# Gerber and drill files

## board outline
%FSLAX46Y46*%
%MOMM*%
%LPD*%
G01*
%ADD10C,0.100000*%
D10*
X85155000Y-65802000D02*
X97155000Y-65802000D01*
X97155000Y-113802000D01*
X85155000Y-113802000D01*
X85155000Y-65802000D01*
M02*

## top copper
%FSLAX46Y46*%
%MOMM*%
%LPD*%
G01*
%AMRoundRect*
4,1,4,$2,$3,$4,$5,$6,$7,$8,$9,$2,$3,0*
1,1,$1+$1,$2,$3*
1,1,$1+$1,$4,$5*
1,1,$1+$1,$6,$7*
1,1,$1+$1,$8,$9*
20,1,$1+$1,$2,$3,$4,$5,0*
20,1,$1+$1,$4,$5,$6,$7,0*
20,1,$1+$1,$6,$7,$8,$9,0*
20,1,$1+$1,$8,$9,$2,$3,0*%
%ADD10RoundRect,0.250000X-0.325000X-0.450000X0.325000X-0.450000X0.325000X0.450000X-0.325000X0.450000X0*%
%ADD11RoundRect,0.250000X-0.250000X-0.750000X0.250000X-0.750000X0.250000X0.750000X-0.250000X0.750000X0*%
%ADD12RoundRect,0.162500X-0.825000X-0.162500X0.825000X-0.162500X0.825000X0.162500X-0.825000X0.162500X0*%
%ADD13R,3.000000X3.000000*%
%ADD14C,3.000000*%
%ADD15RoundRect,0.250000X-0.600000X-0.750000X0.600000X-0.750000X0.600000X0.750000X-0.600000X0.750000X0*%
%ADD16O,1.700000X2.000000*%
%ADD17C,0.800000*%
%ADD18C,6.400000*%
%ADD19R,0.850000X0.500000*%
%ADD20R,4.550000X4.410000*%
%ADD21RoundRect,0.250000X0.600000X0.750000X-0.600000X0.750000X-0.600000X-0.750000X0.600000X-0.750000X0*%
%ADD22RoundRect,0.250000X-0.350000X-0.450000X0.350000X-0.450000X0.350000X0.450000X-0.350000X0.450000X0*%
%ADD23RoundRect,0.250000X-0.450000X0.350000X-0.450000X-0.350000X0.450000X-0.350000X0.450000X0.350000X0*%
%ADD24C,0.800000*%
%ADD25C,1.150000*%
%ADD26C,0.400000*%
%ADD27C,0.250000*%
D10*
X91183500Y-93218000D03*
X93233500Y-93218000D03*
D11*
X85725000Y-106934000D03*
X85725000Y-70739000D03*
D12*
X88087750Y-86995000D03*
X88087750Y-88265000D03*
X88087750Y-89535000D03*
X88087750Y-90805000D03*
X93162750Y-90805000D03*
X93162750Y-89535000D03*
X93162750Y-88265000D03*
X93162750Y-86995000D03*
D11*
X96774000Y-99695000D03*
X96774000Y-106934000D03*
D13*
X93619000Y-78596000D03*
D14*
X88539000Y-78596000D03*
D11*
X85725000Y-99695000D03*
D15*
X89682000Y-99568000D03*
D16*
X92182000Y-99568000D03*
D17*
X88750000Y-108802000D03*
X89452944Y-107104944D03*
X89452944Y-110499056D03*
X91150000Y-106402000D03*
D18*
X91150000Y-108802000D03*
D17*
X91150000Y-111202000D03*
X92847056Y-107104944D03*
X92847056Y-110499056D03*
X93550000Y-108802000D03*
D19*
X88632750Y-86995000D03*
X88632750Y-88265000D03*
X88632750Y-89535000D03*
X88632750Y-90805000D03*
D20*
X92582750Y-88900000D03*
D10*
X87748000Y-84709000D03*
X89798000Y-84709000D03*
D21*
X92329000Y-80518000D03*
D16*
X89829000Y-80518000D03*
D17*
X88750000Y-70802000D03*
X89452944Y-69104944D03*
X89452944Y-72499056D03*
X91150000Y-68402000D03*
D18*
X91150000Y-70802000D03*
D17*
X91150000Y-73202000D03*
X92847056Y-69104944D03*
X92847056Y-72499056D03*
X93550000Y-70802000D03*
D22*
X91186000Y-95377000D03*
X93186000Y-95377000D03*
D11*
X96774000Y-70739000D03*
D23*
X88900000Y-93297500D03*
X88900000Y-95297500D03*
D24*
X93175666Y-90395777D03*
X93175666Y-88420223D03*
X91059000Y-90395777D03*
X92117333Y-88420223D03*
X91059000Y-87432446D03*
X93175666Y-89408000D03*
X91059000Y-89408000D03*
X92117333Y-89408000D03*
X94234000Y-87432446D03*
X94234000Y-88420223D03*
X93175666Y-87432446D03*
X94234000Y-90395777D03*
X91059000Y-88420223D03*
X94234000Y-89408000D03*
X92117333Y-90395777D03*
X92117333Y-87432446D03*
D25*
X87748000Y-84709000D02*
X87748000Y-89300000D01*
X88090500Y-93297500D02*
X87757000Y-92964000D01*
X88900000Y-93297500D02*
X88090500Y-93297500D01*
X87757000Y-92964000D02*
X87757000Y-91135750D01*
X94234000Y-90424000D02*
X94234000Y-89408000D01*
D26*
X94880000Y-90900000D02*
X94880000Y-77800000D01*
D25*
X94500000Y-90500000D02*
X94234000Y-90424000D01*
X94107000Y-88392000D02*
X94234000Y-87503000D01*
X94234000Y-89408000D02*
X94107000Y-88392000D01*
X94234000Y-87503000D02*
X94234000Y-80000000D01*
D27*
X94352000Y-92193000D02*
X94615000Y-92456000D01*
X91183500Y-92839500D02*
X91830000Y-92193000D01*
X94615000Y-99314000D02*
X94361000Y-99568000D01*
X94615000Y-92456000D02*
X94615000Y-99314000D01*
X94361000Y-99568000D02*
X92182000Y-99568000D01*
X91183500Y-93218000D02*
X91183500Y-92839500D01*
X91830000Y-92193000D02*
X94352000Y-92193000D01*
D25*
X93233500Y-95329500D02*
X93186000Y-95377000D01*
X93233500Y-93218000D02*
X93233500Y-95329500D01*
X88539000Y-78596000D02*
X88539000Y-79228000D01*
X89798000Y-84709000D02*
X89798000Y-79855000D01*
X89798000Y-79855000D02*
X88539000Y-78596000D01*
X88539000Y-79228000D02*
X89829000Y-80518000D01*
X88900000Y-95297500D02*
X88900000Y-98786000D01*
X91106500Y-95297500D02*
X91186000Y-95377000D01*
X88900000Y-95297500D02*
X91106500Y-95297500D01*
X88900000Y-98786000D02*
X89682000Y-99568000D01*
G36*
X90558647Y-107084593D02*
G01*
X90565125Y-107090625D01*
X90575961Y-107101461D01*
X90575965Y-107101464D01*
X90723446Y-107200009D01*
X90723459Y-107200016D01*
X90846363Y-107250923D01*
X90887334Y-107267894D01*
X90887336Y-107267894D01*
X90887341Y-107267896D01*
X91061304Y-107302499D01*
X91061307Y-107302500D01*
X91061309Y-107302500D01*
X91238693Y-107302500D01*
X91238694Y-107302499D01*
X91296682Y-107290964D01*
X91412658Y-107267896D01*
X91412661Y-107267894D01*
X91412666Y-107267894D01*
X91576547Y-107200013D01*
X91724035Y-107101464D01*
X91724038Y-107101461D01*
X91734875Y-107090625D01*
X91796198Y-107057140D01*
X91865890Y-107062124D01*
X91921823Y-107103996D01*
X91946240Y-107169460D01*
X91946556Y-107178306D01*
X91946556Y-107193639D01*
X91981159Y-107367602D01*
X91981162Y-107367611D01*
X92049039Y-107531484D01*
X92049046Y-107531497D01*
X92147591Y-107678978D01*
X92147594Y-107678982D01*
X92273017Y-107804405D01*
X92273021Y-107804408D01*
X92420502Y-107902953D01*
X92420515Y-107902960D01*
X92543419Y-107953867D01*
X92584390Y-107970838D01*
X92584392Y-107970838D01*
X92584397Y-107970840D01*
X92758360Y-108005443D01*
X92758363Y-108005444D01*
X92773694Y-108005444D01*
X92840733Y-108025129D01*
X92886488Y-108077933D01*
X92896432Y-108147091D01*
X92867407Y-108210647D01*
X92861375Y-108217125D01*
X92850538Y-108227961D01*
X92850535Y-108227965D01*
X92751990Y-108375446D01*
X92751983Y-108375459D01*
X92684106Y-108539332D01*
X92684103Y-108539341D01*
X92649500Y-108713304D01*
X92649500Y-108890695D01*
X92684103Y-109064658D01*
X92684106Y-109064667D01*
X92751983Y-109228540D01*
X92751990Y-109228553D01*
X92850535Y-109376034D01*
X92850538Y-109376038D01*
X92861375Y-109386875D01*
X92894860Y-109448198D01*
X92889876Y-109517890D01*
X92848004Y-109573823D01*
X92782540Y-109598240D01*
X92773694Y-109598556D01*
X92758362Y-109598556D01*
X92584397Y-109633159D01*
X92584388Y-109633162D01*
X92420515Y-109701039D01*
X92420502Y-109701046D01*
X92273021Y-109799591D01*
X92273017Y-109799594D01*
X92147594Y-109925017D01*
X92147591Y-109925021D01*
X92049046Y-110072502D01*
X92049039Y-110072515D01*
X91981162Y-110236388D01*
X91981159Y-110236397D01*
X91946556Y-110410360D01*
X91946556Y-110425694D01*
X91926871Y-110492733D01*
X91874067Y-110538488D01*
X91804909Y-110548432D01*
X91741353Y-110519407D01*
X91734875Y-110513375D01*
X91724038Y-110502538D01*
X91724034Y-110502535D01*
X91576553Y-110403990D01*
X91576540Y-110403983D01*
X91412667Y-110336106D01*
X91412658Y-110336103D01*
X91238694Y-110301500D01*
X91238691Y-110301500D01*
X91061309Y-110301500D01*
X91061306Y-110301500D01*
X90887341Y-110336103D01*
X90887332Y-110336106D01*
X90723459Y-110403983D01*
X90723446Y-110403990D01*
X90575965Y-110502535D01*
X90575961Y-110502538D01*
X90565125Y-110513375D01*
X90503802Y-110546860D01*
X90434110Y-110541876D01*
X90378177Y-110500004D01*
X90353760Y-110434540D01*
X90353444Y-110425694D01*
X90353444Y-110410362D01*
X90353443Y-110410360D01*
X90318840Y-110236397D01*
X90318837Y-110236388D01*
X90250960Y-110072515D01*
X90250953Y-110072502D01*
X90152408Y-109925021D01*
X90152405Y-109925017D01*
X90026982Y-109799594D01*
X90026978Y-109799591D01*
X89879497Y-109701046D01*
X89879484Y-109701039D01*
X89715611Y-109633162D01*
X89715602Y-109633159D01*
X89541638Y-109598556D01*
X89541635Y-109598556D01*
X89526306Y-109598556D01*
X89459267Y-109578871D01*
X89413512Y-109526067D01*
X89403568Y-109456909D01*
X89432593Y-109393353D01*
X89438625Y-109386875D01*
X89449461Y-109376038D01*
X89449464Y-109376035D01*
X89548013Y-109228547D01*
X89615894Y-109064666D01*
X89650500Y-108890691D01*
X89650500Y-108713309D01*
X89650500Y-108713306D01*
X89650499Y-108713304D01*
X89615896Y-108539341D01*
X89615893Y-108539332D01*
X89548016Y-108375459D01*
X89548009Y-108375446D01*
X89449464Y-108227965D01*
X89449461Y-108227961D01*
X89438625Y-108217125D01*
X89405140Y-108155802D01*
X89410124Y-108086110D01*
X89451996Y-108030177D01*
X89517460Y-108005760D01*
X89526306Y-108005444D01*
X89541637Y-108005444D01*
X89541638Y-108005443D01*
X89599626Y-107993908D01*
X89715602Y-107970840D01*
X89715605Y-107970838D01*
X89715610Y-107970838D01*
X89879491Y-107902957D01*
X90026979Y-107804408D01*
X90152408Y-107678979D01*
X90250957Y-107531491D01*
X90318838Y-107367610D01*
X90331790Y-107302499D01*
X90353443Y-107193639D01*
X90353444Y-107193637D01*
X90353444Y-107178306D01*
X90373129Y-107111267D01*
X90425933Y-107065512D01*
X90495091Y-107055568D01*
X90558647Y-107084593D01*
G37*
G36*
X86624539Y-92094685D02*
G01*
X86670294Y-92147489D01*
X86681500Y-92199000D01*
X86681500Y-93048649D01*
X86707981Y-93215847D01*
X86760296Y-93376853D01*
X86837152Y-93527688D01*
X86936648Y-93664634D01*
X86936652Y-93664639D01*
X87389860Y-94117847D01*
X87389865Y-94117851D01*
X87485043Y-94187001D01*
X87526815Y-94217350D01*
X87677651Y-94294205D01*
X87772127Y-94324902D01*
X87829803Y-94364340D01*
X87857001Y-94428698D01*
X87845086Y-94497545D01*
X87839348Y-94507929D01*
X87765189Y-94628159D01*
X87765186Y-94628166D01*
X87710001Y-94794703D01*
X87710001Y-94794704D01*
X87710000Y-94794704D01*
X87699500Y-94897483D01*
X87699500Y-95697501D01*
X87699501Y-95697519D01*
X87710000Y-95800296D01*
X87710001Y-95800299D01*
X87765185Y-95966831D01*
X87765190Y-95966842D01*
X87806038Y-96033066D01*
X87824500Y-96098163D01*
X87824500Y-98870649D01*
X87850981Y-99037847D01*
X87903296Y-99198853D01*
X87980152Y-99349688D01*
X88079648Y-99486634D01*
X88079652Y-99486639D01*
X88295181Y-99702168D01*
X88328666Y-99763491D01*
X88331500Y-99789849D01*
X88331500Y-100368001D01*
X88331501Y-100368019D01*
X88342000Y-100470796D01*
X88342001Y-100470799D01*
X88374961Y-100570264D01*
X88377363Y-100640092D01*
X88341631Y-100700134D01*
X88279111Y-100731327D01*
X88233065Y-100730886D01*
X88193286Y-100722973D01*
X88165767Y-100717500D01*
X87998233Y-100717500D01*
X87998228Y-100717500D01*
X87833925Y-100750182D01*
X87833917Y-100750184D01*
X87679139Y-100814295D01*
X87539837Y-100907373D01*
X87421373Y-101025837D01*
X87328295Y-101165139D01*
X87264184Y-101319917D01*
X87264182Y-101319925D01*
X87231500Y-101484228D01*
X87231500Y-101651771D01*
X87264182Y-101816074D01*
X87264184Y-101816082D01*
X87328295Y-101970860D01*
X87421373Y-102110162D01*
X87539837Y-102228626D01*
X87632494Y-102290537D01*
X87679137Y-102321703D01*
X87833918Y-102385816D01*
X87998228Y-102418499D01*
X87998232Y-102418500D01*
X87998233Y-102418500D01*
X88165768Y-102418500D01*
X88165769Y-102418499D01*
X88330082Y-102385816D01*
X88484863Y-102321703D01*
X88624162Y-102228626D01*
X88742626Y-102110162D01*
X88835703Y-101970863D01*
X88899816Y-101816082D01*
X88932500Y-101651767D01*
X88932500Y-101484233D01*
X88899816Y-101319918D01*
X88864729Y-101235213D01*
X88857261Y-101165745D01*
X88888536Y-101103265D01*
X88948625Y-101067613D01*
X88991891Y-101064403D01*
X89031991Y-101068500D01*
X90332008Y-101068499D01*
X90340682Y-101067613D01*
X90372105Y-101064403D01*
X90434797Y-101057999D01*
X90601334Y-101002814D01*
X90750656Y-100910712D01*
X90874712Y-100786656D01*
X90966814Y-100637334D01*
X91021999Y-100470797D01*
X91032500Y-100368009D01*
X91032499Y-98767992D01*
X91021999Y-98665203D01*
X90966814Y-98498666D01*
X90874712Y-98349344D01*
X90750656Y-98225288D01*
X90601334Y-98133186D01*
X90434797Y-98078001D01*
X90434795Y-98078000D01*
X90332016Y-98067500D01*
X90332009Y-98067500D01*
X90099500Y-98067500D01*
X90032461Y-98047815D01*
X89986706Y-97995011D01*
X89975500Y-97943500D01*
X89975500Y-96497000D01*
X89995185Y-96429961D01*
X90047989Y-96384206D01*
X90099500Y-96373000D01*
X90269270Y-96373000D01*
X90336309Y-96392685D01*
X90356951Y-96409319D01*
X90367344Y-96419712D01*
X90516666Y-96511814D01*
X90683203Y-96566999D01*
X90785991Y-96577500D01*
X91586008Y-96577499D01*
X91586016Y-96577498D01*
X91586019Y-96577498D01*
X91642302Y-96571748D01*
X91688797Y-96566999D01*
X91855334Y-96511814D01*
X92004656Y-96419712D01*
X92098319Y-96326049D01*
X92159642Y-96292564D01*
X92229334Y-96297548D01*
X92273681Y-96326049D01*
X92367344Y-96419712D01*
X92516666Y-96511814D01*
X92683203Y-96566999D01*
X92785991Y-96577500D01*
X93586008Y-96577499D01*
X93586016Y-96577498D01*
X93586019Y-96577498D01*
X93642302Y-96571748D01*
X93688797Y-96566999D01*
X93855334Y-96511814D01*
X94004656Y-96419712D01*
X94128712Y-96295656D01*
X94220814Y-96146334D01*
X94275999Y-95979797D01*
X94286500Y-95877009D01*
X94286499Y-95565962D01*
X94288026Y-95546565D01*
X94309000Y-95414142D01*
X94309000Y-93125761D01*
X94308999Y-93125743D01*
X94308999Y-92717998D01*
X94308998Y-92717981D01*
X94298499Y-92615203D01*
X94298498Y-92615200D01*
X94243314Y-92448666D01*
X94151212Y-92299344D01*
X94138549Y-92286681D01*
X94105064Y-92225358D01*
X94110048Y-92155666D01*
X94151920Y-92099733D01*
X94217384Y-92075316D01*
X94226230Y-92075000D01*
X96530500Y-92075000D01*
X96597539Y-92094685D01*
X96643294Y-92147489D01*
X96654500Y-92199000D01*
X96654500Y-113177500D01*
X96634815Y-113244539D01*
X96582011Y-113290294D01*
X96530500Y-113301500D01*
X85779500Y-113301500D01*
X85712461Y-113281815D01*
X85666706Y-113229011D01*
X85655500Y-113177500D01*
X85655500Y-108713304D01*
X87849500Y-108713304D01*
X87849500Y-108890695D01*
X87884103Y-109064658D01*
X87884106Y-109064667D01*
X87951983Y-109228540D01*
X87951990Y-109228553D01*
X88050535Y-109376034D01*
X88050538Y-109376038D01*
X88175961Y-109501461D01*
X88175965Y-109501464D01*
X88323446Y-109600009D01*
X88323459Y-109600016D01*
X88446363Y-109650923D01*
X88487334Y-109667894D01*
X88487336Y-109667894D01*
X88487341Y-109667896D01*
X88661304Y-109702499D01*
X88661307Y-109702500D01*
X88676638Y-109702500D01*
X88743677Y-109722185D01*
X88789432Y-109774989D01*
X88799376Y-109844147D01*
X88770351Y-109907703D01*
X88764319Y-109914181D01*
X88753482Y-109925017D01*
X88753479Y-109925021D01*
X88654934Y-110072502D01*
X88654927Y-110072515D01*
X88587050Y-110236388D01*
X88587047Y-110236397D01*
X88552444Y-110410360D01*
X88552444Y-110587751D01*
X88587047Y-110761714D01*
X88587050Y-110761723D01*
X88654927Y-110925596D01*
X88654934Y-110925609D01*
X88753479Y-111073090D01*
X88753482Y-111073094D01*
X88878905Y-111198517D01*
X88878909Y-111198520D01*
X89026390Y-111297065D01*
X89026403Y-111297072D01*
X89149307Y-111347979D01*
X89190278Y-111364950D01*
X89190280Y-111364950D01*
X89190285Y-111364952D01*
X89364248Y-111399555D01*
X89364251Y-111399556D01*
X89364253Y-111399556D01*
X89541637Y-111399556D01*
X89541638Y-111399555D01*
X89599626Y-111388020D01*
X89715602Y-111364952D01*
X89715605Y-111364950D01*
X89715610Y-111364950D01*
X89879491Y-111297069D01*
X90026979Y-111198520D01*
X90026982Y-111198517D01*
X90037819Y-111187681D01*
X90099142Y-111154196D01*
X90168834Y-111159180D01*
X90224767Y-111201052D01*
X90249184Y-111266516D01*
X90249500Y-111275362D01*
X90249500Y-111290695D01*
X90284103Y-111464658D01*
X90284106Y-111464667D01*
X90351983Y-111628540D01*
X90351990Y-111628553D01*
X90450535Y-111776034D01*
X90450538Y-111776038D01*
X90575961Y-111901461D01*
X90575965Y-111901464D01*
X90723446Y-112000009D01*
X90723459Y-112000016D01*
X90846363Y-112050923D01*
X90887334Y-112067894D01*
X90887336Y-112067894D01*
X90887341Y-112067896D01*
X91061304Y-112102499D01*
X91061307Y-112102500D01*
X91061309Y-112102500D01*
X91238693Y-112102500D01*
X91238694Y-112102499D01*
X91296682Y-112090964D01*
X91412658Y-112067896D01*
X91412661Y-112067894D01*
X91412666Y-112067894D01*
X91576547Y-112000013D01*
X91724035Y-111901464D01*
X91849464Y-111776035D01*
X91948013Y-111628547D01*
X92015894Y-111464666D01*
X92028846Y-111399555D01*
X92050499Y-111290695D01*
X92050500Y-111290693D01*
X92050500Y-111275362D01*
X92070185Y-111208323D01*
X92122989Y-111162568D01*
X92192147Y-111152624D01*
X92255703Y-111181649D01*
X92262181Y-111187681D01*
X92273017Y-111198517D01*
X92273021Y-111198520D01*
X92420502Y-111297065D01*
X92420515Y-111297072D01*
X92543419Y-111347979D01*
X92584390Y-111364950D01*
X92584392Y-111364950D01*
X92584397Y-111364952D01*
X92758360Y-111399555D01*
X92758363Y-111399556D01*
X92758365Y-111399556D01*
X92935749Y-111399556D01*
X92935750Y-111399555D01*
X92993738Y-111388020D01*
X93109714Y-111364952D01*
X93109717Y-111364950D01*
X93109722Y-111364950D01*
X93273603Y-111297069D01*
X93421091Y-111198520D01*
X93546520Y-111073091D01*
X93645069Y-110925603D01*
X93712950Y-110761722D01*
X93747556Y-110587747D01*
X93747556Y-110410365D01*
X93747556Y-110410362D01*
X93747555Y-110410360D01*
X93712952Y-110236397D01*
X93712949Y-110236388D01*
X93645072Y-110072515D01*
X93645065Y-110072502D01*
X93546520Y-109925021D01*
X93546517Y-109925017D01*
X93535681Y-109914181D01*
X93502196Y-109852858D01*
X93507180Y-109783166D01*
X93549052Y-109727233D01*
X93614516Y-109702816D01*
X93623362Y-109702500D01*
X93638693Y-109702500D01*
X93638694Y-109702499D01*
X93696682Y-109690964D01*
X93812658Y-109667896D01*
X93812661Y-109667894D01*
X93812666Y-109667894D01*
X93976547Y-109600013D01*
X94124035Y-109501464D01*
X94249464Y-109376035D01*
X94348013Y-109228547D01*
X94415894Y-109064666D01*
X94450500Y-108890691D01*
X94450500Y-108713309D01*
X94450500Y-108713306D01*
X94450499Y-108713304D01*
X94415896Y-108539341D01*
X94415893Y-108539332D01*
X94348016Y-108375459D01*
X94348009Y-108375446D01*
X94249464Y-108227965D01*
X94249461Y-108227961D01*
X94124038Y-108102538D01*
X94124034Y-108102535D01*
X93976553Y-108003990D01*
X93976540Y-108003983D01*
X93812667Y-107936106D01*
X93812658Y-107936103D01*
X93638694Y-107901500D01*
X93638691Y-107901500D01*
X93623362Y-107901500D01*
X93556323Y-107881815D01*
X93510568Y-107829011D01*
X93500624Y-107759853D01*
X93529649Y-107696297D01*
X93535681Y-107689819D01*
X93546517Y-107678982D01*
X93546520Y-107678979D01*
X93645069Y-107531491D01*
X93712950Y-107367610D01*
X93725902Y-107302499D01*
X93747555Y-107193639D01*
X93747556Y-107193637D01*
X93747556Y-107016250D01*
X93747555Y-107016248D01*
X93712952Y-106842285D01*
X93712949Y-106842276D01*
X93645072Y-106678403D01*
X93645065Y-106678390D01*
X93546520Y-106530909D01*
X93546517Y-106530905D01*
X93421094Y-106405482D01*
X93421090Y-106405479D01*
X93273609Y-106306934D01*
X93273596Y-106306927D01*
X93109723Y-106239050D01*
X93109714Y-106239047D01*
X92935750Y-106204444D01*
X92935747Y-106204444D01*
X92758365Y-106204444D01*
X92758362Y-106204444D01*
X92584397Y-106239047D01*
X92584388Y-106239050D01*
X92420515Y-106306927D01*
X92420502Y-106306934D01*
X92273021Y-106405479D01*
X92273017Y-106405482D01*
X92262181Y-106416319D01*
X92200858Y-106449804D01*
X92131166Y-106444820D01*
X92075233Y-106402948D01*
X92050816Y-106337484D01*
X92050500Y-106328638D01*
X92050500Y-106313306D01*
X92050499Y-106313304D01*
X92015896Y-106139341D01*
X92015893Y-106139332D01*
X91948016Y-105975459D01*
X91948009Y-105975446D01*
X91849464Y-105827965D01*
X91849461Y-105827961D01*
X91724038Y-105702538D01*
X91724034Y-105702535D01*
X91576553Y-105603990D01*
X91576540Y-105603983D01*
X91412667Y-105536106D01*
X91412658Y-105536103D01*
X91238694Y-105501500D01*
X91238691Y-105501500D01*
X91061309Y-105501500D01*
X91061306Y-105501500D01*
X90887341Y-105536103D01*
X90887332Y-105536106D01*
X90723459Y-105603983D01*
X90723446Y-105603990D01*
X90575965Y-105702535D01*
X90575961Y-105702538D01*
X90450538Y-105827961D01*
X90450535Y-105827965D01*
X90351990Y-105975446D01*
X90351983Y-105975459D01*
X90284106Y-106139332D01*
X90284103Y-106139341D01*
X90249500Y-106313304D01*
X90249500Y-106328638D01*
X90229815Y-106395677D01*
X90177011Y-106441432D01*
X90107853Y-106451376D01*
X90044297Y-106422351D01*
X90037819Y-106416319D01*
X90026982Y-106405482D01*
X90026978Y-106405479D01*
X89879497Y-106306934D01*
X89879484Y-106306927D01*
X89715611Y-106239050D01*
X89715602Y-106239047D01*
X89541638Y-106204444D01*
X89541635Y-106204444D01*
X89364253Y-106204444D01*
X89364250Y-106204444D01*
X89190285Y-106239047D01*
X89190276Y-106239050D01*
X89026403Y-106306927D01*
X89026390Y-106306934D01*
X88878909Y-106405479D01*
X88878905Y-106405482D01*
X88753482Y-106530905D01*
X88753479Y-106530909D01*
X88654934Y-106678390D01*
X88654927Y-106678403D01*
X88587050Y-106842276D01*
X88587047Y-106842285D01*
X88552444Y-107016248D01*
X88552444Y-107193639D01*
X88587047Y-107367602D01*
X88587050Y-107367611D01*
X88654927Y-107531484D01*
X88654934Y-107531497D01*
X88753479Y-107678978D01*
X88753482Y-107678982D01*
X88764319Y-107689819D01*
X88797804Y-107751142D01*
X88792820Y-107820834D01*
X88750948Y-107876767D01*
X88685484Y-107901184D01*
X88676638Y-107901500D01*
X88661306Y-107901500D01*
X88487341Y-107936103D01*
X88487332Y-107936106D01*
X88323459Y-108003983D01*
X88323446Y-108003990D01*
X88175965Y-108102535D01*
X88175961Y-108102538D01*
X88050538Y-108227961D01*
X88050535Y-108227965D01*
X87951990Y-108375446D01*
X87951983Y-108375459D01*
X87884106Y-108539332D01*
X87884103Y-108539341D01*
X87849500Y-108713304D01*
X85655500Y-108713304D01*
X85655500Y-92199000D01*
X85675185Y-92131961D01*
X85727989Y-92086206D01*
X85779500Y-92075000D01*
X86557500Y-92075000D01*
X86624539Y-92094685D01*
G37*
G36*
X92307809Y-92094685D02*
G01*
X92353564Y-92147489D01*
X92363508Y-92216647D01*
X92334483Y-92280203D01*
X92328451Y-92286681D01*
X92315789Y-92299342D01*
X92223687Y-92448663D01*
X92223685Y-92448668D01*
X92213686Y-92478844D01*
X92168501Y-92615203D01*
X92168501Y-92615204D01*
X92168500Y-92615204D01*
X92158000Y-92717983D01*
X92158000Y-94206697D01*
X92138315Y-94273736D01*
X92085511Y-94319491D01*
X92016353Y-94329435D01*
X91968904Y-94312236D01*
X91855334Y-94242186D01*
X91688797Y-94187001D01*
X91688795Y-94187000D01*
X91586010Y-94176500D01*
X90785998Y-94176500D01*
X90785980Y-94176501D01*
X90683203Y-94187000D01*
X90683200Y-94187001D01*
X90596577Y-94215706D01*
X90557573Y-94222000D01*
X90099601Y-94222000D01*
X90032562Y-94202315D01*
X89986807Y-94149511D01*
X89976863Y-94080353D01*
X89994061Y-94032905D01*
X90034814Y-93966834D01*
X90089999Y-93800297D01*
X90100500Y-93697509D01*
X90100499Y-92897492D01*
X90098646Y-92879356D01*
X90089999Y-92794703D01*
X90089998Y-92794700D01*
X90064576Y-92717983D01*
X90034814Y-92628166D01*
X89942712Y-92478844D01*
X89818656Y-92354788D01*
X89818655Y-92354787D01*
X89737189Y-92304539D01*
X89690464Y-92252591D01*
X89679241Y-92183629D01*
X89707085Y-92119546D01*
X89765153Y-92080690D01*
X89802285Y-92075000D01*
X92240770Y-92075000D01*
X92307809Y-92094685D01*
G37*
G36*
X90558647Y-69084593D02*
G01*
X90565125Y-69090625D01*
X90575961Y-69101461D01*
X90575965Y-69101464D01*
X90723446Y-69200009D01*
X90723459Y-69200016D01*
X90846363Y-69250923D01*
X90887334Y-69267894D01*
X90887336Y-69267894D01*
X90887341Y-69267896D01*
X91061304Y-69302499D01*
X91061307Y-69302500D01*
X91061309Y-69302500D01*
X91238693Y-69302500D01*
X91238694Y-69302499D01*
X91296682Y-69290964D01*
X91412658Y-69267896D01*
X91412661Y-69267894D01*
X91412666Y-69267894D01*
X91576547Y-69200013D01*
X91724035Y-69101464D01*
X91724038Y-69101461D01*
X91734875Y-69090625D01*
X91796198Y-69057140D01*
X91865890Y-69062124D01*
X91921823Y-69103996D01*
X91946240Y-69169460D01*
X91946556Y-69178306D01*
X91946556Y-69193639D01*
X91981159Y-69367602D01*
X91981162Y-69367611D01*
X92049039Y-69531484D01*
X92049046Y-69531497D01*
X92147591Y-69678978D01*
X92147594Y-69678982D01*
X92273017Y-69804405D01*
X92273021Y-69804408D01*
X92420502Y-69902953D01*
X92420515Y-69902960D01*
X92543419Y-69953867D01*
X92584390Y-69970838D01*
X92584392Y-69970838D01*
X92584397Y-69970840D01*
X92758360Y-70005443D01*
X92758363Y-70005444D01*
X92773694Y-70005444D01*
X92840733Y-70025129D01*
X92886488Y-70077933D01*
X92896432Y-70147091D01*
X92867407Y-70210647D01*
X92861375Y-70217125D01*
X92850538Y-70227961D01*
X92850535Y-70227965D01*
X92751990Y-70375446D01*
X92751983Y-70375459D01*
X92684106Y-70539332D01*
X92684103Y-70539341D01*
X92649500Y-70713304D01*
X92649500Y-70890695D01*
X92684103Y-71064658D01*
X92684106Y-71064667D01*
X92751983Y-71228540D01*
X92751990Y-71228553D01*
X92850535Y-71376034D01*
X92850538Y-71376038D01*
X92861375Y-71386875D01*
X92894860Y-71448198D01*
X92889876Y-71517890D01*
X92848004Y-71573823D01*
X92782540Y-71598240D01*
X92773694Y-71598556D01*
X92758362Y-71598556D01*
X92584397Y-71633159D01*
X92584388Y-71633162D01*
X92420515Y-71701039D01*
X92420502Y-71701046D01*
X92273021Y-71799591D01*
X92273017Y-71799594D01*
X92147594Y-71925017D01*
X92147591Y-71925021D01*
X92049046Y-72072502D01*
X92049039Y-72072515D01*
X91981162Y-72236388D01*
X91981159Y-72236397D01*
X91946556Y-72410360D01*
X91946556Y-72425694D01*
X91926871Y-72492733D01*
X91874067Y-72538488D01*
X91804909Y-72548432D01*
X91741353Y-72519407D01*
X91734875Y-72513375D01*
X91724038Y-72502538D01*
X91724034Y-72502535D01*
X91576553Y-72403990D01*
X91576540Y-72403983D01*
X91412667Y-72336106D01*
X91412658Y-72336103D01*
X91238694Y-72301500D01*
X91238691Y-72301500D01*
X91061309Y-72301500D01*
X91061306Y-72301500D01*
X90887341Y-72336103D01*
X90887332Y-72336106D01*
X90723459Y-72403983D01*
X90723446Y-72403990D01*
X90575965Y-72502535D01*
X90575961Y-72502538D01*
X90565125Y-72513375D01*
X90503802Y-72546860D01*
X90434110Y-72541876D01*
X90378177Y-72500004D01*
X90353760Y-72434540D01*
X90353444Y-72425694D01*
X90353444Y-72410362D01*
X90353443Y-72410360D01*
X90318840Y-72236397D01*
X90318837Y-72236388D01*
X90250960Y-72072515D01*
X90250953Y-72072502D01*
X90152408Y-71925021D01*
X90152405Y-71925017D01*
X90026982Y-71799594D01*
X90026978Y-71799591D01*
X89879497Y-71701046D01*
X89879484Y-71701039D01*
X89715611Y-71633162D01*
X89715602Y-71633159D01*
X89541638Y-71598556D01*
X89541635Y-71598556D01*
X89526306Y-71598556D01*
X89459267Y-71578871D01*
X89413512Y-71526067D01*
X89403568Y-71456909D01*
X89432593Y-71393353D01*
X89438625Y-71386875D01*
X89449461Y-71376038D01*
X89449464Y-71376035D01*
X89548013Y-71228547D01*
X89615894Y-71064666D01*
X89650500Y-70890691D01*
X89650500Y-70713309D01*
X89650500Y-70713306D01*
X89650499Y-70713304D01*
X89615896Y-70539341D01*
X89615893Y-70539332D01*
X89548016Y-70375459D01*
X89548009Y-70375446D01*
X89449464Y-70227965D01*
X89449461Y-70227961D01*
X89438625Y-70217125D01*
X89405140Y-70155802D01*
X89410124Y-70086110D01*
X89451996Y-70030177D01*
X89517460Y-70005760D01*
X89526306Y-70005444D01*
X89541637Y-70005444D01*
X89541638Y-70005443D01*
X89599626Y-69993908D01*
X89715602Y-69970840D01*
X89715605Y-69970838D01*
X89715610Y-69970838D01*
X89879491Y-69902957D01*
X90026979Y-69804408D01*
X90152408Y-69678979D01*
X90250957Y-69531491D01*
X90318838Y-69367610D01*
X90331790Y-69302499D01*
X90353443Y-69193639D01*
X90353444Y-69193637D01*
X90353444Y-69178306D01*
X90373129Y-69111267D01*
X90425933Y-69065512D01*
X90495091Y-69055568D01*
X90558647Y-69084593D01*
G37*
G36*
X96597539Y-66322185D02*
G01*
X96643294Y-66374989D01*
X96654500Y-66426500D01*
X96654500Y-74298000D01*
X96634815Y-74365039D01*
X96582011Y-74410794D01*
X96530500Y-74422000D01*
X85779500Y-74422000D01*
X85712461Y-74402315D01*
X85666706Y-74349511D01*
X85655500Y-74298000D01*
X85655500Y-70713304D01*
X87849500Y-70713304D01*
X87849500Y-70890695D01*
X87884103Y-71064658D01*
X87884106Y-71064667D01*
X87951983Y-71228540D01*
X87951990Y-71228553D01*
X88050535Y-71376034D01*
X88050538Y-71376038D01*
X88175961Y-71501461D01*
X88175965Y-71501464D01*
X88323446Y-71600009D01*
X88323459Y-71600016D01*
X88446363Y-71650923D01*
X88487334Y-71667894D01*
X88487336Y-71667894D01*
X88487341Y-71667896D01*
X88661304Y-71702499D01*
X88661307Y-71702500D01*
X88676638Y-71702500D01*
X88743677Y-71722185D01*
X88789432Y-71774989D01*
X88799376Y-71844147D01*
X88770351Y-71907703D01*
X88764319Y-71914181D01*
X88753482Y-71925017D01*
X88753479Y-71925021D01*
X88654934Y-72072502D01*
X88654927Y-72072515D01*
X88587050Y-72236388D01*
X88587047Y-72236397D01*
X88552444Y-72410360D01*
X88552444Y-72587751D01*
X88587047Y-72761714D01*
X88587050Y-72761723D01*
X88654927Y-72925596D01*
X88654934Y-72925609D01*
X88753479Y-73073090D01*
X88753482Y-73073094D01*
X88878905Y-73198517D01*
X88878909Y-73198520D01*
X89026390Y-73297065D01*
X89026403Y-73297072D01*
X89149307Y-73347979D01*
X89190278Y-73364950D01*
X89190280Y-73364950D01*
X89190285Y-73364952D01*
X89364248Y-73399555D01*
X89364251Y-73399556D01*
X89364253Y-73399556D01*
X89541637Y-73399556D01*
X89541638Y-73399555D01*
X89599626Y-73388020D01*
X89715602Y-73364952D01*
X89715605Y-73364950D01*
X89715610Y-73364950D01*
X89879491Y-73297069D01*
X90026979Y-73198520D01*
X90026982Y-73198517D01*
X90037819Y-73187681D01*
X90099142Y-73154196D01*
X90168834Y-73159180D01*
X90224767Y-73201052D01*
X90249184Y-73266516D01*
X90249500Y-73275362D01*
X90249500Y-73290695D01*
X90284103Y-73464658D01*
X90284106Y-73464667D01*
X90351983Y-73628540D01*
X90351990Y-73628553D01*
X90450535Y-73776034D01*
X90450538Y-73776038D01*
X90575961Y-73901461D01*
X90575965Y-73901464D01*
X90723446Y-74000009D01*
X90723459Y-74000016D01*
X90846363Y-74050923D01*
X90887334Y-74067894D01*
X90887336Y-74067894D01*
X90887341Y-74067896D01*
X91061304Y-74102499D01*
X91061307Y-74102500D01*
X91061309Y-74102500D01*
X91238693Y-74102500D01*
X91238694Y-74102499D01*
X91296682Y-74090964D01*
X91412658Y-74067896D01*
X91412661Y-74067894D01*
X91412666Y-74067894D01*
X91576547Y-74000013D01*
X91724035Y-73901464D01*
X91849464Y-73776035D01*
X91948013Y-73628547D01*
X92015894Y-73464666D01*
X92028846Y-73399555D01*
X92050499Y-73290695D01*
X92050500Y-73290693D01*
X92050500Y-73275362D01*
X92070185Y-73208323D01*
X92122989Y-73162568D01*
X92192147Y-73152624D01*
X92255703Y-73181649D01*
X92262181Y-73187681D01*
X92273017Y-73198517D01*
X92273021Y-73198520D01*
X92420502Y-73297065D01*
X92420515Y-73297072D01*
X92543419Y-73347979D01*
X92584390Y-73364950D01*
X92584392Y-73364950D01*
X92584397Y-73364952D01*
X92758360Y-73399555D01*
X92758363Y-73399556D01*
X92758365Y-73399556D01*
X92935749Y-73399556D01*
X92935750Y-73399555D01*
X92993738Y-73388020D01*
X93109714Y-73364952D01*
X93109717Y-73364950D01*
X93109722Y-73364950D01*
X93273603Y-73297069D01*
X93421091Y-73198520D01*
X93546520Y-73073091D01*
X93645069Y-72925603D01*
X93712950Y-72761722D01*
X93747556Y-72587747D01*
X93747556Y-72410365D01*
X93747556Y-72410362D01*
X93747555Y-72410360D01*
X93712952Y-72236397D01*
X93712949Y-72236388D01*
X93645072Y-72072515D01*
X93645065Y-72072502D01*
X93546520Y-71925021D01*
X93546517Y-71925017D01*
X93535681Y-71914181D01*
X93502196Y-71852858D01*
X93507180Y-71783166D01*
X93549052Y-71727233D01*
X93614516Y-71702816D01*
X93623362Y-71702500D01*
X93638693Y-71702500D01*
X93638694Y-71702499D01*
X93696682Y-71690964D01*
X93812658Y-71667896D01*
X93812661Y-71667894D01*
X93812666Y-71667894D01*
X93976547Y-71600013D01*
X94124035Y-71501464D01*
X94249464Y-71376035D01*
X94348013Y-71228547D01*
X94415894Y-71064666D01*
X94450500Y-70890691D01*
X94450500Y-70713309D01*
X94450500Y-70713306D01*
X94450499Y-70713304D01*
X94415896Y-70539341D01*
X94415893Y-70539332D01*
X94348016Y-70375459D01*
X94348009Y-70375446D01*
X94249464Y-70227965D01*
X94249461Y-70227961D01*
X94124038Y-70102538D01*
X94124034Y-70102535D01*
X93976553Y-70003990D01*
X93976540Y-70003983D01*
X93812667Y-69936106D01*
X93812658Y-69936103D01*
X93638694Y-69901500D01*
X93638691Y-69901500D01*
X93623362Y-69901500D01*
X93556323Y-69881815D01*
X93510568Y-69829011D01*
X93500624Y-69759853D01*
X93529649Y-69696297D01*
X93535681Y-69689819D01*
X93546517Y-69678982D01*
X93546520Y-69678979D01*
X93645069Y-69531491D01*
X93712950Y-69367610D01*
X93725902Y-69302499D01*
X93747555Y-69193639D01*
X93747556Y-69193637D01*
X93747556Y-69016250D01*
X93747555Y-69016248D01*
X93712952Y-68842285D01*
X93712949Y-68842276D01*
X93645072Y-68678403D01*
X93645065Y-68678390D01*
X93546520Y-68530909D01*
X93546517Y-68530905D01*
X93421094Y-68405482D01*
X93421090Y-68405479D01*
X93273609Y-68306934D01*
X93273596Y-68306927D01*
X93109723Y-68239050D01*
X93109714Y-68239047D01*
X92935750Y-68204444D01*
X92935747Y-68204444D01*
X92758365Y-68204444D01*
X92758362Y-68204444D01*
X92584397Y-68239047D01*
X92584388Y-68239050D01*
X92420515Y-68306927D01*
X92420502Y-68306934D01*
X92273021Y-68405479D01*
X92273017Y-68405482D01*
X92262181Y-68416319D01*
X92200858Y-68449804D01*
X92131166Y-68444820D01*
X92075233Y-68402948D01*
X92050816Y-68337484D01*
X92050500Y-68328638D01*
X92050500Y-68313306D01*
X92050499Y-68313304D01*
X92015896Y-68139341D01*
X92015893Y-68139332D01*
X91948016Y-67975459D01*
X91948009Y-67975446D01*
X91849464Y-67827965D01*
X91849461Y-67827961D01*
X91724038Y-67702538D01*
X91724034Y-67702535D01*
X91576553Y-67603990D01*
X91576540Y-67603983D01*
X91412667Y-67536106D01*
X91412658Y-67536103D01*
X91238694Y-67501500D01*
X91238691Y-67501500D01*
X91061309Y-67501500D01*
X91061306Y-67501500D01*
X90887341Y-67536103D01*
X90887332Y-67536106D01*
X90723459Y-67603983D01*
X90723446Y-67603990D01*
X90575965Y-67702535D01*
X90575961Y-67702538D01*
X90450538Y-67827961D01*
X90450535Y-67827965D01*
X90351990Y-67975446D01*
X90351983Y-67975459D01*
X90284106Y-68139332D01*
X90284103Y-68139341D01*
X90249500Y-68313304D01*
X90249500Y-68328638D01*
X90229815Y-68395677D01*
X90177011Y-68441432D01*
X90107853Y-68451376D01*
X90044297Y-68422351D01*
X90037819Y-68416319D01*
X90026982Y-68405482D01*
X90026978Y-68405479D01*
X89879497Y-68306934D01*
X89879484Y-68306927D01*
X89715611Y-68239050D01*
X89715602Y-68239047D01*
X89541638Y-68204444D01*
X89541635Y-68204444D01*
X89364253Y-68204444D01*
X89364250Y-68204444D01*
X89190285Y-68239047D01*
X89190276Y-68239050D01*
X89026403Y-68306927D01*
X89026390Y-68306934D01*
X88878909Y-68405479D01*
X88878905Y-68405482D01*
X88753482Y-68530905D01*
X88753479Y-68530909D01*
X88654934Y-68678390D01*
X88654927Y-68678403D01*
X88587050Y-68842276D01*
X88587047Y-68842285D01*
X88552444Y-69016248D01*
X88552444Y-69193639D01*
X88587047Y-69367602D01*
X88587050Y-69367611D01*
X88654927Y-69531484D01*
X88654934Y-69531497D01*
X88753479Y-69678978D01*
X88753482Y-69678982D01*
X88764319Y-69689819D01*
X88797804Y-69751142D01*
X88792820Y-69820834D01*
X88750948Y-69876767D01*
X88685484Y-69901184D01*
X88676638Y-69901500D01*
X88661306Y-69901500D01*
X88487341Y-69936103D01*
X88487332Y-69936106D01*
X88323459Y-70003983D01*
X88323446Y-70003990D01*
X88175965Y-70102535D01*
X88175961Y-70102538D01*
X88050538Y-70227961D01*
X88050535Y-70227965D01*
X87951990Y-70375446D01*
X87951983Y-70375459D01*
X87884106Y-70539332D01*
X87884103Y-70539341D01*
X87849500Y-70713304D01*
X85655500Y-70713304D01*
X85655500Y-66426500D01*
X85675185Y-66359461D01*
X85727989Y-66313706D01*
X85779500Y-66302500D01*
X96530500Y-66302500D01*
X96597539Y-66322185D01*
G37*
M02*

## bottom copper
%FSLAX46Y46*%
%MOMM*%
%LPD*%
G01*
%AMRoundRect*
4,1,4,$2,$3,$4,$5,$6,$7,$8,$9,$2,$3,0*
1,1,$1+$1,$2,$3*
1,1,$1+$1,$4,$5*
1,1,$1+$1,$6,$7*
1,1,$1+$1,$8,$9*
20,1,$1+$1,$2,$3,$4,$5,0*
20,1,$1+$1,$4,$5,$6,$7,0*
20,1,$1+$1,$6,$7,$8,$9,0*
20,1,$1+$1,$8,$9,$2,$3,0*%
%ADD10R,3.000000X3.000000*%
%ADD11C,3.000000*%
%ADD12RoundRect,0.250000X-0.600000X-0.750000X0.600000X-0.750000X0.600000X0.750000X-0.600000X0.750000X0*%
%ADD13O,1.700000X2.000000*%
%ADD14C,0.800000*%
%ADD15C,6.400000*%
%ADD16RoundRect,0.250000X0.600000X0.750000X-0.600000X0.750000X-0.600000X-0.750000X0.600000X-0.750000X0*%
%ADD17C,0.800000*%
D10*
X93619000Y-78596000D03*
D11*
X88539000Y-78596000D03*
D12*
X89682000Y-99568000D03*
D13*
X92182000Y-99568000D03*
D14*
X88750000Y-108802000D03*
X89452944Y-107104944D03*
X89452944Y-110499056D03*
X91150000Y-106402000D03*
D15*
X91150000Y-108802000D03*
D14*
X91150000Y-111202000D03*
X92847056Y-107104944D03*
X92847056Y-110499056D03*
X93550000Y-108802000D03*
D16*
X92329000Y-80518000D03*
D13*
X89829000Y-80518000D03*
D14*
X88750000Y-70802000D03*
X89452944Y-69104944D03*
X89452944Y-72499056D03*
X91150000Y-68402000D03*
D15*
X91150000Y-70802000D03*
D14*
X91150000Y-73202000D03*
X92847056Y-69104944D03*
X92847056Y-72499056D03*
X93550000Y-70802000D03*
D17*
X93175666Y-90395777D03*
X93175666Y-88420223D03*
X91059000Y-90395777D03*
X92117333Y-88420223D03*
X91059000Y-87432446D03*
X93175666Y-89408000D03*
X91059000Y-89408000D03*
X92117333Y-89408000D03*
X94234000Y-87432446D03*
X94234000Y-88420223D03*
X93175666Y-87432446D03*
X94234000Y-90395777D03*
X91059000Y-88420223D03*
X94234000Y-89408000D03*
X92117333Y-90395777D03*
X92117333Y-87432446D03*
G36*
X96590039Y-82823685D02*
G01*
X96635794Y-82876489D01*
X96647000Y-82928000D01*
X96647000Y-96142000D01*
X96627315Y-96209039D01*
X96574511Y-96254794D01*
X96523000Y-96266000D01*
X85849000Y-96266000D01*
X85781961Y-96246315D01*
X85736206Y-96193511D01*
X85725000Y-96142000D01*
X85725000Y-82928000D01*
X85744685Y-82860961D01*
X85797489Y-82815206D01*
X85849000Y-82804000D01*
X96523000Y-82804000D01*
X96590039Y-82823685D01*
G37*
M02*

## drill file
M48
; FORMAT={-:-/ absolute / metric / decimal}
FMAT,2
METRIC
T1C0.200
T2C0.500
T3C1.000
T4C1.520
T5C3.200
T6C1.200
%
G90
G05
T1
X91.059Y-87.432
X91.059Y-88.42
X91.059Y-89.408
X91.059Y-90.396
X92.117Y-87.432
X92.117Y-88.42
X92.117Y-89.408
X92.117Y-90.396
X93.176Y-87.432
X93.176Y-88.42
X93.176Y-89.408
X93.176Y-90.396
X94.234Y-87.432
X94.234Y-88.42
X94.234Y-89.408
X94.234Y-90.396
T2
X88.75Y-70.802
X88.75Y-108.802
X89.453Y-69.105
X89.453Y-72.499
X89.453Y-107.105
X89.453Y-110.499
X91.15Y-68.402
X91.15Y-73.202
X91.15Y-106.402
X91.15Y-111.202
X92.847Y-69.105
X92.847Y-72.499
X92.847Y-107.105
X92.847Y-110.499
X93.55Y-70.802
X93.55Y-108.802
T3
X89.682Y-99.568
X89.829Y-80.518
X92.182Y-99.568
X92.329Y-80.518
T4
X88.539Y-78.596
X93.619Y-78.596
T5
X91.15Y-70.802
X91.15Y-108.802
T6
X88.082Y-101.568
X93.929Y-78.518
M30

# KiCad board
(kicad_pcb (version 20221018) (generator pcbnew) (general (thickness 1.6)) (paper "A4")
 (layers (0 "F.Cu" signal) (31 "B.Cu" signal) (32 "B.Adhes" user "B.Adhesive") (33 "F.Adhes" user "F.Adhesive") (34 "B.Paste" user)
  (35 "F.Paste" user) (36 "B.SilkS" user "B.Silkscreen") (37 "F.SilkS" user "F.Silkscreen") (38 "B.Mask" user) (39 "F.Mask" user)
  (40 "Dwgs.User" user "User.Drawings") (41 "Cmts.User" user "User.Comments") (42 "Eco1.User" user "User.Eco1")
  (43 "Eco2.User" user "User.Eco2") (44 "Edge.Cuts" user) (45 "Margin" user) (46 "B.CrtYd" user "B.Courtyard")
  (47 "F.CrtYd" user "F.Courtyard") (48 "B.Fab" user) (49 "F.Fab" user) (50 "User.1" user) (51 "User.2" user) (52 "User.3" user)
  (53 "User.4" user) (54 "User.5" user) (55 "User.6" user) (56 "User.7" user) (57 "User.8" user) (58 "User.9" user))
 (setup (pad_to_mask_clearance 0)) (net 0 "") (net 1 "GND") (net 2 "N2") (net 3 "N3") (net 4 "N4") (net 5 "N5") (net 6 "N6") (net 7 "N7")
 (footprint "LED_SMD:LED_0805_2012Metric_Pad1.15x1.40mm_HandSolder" (layer "F.Cu") (at 92.2085 93.218)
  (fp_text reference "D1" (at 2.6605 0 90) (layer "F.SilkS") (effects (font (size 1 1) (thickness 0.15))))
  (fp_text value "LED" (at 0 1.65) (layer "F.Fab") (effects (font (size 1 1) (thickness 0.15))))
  (pad "1" smd roundrect (at -1.025 0) (size 1.15 1.4) (layers "F.Cu" "F.Paste" "F.Mask") (roundrect_rratio 0.217391) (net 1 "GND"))
  (pad "2" smd roundrect (at 1.025 0) (size 1.15 1.4) (layers "F.Cu" "F.Paste" "F.Mask") (roundrect_rratio 0.217391) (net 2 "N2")))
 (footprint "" (layer "F.Cu") (at 85.725 106.934)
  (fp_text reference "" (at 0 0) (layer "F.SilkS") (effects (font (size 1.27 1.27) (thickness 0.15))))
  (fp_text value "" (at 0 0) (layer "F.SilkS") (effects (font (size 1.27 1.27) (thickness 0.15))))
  (pad "1" smd roundrect (at 0 0) (size 1 2) (layers "F.Cu" "F.Paste" "F.Mask") (roundrect_rratio 0.25) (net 1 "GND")))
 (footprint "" (layer "F.Cu") (at 85.725 70.739)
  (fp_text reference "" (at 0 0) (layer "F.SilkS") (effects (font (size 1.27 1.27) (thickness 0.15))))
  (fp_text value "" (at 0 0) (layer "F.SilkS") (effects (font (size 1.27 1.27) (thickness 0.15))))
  (pad "1" smd roundrect (at 0 0) (size 1 2) (layers "F.Cu" "F.Paste" "F.Mask") (roundrect_rratio 0.25) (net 1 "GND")))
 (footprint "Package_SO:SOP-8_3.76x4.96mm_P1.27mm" (layer "F.Cu") (at 90.62525 88.9)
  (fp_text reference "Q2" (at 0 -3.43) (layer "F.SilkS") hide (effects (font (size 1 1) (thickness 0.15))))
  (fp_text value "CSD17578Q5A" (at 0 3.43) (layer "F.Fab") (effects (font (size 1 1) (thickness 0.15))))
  (pad "1" smd roundrect (at -2.5375 -1.905) (size 1.975 0.65) (layers "F.Cu" "F.Paste" "F.Mask") (roundrect_rratio 0.25) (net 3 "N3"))
  (pad "2" smd roundrect (at -2.5375 -0.635) (size 1.975 0.65) (layers "F.Cu" "F.Paste" "F.Mask") (roundrect_rratio 0.25) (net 3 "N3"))
  (pad "3" smd roundrect (at -2.5375 0.635) (size 1.975 0.65) (layers "F.Cu" "F.Paste" "F.Mask") (roundrect_rratio 0.25) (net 3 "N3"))
  (pad "4" smd roundrect (at -2.5375 1.905) (size 1.975 0.65) (layers "F.Cu" "F.Paste" "F.Mask") (roundrect_rratio 0.25) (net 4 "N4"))
  (pad "5" smd roundrect (at 2.5375 1.905) (size 1.975 0.65) (layers "F.Cu" "F.Paste" "F.Mask") (roundrect_rratio 0.25) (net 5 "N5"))
  (pad "6" smd roundrect (at 2.5375 0.635) (size 1.975 0.65) (layers "F.Cu" "F.Paste" "F.Mask") (roundrect_rratio 0.25) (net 5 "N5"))
  (pad "7" smd roundrect (at 2.5375 -0.635) (size 1.975 0.65) (layers "F.Cu" "F.Paste" "F.Mask") (roundrect_rratio 0.25) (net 5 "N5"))
  (pad "8" smd roundrect (at 2.5375 -1.905) (size 1.975 0.65) (layers "F.Cu" "F.Paste" "F.Mask") (roundrect_rratio 0.25) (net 5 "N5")))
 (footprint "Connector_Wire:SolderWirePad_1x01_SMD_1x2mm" (layer "F.Cu") (at 96.774 99.695)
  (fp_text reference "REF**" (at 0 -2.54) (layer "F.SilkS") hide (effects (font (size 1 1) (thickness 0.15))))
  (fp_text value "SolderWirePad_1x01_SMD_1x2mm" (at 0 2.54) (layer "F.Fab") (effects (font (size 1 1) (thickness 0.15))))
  (pad "1" smd roundrect (at 0 0) (size 1 2) (layers "F.Cu" "F.Paste" "F.Mask") (roundrect_rratio 0.25) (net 1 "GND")))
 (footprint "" (layer "F.Cu") (at 96.774 106.934)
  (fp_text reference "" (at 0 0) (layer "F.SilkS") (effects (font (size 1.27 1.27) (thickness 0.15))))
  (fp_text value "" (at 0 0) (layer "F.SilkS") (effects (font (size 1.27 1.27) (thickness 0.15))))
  (pad "1" smd roundrect (at 0 0) (size 1 2) (layers "F.Cu" "F.Paste" "F.Mask") (roundrect_rratio 0.25) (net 1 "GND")))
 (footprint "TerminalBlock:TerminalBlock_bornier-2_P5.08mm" (layer "F.Cu") (at 93.619 78.596 180)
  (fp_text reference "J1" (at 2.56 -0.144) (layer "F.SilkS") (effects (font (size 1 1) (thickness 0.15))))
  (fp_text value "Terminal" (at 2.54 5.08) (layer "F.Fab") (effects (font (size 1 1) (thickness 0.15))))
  (pad "1" thru_hole rect (at 0 0 180) (size 3 3) (drill 1.52) (layers "*.Cu" "*.Mask") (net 5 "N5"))
  (pad "2" thru_hole circle (at 5.08 0 180) (size 3 3) (drill 1.52) (layers "*.Cu" "*.Mask") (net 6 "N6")))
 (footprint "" (layer "F.Cu") (at 85.725 99.695)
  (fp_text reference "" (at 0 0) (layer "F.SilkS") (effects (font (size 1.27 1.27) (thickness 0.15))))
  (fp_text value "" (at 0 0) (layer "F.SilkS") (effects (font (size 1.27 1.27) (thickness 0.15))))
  (pad "1" smd roundrect (at 0 0) (size 1 2) (layers "F.Cu" "F.Paste" "F.Mask") (roundrect_rratio 0.25) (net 1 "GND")))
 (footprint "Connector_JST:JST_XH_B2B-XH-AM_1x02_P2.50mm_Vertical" (layer "F.Cu") (at 89.682 99.568)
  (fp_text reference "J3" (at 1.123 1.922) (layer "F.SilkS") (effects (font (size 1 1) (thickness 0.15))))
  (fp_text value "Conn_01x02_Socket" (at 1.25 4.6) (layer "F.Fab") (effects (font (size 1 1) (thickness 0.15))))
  (pad "" np_thru_hole circle (at -1.6 2) (size 1.2 1.2) (drill 1.2) (layers "*.Cu" "*.Mask"))
  (pad "1" thru_hole roundrect (at 0 0) (size 1.7 2) (drill 1) (layers "*.Cu" "*.Mask") (roundrect_rratio 0.147059) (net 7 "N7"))
  (pad "2" thru_hole oval (at 2.5 0) (size 1.7 2) (drill 1) (layers "*.Cu" "*.Mask") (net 1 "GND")))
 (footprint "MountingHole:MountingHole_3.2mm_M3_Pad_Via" (layer "F.Cu") (at 91.15 108.802)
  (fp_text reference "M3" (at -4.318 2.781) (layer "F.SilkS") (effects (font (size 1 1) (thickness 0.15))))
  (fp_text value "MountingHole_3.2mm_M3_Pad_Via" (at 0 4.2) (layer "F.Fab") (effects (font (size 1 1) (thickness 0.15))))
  (pad "1" thru_hole circle (at -2.4 0) (size 0.8 0.8) (drill 0.5) (layers "*.Cu" "*.Mask"))
  (pad "1" thru_hole circle (at -1.697056 -1.697056) (size 0.8 0.8) (drill 0.5) (layers "*.Cu" "*.Mask"))
  (pad "1" thru_hole circle (at -1.697056 1.697056) (size 0.8 0.8) (drill 0.5) (layers "*.Cu" "*.Mask"))
  (pad "1" thru_hole circle (at 0 -2.4) (size 0.8 0.8) (drill 0.5) (layers "*.Cu" "*.Mask"))
  (pad "1" thru_hole circle (at 0 0) (size 6.4 6.4) (drill 3.2) (layers "*.Cu" "*.Mask") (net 1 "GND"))
  (pad "1" thru_hole circle (at 0 2.4) (size 0.8 0.8) (drill 0.5) (layers "*.Cu" "*.Mask"))
  (pad "1" thru_hole circle (at 1.697056 -1.697056) (size 0.8 0.8) (drill 0.5) (layers "*.Cu" "*.Mask"))
  (pad "1" thru_hole circle (at 1.697056 1.697056) (size 0.8 0.8) (drill 0.5) (layers "*.Cu" "*.Mask"))
  (pad "1" thru_hole circle (at 2.4 0) (size 0.8 0.8) (drill 0.5) (layers "*.Cu" "*.Mask")))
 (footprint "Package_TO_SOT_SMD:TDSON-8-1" (layer "F.Cu") (at 91.53275 88.9)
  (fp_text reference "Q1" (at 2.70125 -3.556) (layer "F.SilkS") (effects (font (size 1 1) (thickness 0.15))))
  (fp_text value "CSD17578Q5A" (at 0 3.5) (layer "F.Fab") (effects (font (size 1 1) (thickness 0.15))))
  (pad "" smd rect (at -0.2 -0.85) (size 1.5 1.5) (layers "F.Paste"))
  (pad "" smd rect (at -0.2 0.85) (size 1.5 1.5) (layers "F.Paste"))
  (pad "" smd custom (at 0.65 0) (size 3.75 4.41) (layers "F.Mask") (zone_connect 0) (thermal_bridge_angle 45)
   (options (clearance outline) (anchor rect)) (primitives))
  (pad "" smd rect (at 1.5 -0.85) (size 1.5 1.5) (layers "F.Paste"))
  (pad "" smd rect (at 1.5 0.85) (size 1.5 1.5) (layers "F.Paste"))
  (pad "" smd rect (at 2.905 -1.905) (size 0.75 0.5) (layers "F.Paste"))
  (pad "" smd rect (at 2.905 -0.635) (size 0.75 0.5) (layers "F.Paste"))
  (pad "" smd rect (at 2.905 0.635) (size 0.75 0.5) (layers "F.Paste"))
  (pad "" smd rect (at 2.905 1.905) (size 0.75 0.5) (layers "F.Paste"))
  (pad "1" smd rect (at -2.9 -1.905) (size 0.85 0.5) (layers "F.Cu" "F.Paste" "F.Mask") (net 3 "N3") (solder_paste_margin -0.05))
  (pad "2" smd rect (at -2.9 -0.635) (size 0.85 0.5) (layers "F.Cu" "F.Paste" "F.Mask") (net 3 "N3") (solder_paste_margin -0.05))
  (pad "3" smd rect (at -2.9 0.635) (size 0.85 0.5) (layers "F.Cu" "F.Paste" "F.Mask") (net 3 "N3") (solder_paste_margin -0.05))
  (pad "4" smd rect (at -2.9 1.905) (size 0.85 0.5) (layers "F.Cu" "F.Paste" "F.Mask") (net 4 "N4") (solder_paste_margin -0.05))
  (pad "5" smd rect (at 1.05 0) (size 4.55 4.41) (layers "F.Cu") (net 5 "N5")))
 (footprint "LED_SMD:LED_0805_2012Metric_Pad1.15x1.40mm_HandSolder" (layer "F.Cu") (at 88.773 84.709)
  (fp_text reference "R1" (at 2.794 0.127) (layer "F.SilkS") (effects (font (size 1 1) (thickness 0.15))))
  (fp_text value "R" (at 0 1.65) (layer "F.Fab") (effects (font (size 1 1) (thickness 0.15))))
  (pad "1" smd roundrect (at -1.025 0) (size 1.15 1.4) (layers "F.Cu" "F.Paste" "F.Mask") (roundrect_rratio 0.217391) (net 3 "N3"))
  (pad "2" smd roundrect (at 1.025 0) (size 1.15 1.4) (layers "F.Cu" "F.Paste" "F.Mask") (roundrect_rratio 0.217391) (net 6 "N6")))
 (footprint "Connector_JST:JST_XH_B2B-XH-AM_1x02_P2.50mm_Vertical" (layer "F.Cu") (at 92.329 80.518 180)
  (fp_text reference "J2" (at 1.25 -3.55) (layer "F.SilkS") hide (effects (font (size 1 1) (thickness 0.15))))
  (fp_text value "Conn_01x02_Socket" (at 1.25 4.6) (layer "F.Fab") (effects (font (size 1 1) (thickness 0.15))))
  (pad "" np_thru_hole circle (at -1.6 2 180) (size 1.2 1.2) (drill 1.2) (layers "*.Cu" "*.Mask"))
  (pad "1" thru_hole roundrect (at 0 0 180) (size 1.7 2) (drill 1) (layers "*.Cu" "*.Mask") (roundrect_rratio 0.147059) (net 5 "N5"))
  (pad "2" thru_hole oval (at 2.5 0 180) (size 1.7 2) (drill 1) (layers "*.Cu" "*.Mask") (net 6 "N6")))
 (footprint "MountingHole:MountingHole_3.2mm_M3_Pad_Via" (layer "F.Cu") (at 91.15 70.802)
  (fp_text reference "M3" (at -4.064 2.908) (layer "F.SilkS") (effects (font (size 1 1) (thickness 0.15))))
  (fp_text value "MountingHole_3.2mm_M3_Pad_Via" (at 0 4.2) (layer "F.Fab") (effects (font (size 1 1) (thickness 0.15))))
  (pad "1" thru_hole circle (at -2.4 0) (size 0.8 0.8) (drill 0.5) (layers "*.Cu" "*.Mask"))
  (pad "1" thru_hole circle (at -1.697056 -1.697056) (size 0.8 0.8) (drill 0.5) (layers "*.Cu" "*.Mask"))
  (pad "1" thru_hole circle (at -1.697056 1.697056) (size 0.8 0.8) (drill 0.5) (layers "*.Cu" "*.Mask"))
  (pad "1" thru_hole circle (at 0 -2.4) (size 0.8 0.8) (drill 0.5) (layers "*.Cu" "*.Mask"))
  (pad "1" thru_hole circle (at 0 0) (size 6.4 6.4) (drill 3.2) (layers "*.Cu" "*.Mask") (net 1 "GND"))
  (pad "1" thru_hole circle (at 0 2.4) (size 0.8 0.8) (drill 0.5) (layers "*.Cu" "*.Mask"))
  (pad "1" thru_hole circle (at 1.697056 -1.697056) (size 0.8 0.8) (drill 0.5) (layers "*.Cu" "*.Mask"))
  (pad "1" thru_hole circle (at 1.697056 1.697056) (size 0.8 0.8) (drill 0.5) (layers "*.Cu" "*.Mask"))
  (pad "1" thru_hole circle (at 2.4 0) (size 0.8 0.8) (drill 0.5) (layers "*.Cu" "*.Mask")))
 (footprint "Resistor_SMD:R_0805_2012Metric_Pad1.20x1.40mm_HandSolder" (layer "F.Cu") (at 92.186 95.377)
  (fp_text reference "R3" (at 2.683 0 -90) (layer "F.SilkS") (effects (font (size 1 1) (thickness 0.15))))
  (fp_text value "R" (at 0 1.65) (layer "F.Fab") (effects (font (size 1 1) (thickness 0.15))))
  (pad "1" smd roundrect (at -1 0) (size 1.2 1.4) (layers "F.Cu" "F.Paste" "F.Mask") (roundrect_rratio 0.208333) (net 7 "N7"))
  (pad "2" smd roundrect (at 1 0) (size 1.2 1.4) (layers "F.Cu" "F.Paste" "F.Mask") (roundrect_rratio 0.208333) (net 2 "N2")))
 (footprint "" (layer "F.Cu") (at 96.774 70.739)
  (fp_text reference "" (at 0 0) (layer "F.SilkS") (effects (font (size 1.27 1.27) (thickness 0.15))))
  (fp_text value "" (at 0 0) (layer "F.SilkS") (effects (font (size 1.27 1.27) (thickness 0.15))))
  (pad "1" smd roundrect (at 0 0) (size 1 2) (layers "F.Cu" "F.Paste" "F.Mask") (roundrect_rratio 0.25) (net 1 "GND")))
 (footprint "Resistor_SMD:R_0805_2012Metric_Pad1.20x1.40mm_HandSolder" (layer "F.Cu") (at 88.9 94.2975 -90)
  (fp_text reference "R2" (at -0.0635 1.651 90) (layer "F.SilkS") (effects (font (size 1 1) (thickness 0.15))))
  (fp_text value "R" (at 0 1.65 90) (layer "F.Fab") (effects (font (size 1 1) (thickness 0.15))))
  (pad "1" smd roundrect (at -1 0 270) (size 1.2 1.4) (layers "F.Cu" "F.Paste" "F.Mask") (roundrect_rratio 0.208333) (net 4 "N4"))
  (pad "2" smd roundrect (at 1 0 270) (size 1.2 1.4) (layers "F.Cu" "F.Paste" "F.Mask") (roundrect_rratio 0.208333) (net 7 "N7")))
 (gr_rect (start 85.155 65.802) (end 97.155 113.802) (stroke (width 0.1) (type default)) (fill none) (layer "Edge.Cuts"))
 (segment (start 87.748 84.709) (end 87.748 89.3) (width 1.15) (layer "F.Cu") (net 3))
 (segment (start 88.0905 93.2975) (end 87.757 92.964) (width 1.15) (layer "F.Cu") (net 4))
 (segment (start 88.9 93.2975) (end 88.0905 93.2975) (width 1.15) (layer "F.Cu") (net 4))
 (segment (start 87.757 92.964) (end 87.757 91.13575) (width 1.15) (layer "F.Cu") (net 4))
 (segment (start 94.234 90.424) (end 94.234 89.408) (width 1.15) (layer "F.Cu") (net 5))
 (segment (start 94.88 90.9) (end 94.88 77.8) (width 0.4) (layer "F.Cu") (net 5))
 (segment (start 94.5 90.5) (end 94.234 90.424) (width 1.15) (layer "F.Cu") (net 5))
 (segment (start 94.107 88.392) (end 94.234 87.503) (width 1.15) (layer "F.Cu") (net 5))
 (segment (start 94.234 89.408) (end 94.107 88.392) (width 1.15) (layer "F.Cu") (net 5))
 (segment (start 94.234 87.503) (end 94.234 80) (width 1.15) (layer "F.Cu") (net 5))
 (via (at 93.175666 90.395777) (size 0.8) (drill 0.2) (layers "F.Cu" "B.Cu") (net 5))
 (via (at 93.175666 88.420223) (size 0.8) (drill 0.2) (layers "F.Cu" "B.Cu") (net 5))
 (via (at 91.059 90.395777) (size 0.8) (drill 0.2) (layers "F.Cu" "B.Cu") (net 5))
 (via (at 92.117333 88.420223) (size 0.8) (drill 0.2) (layers "F.Cu" "B.Cu") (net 5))
 (via (at 91.059 87.432446) (size 0.8) (drill 0.2) (layers "F.Cu" "B.Cu") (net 5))
 (via (at 93.175666 89.408) (size 0.8) (drill 0.2) (layers "F.Cu" "B.Cu") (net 5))
 (via (at 91.059 89.408) (size 0.8) (drill 0.2) (layers "F.Cu" "B.Cu") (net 5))
 (via (at 92.117333 89.408) (size 0.8) (drill 0.2) (layers "F.Cu" "B.Cu") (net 5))
 (via (at 94.234 87.432446) (size 0.8) (drill 0.2) (layers "F.Cu" "B.Cu") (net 5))
 (via (at 94.234 88.420223) (size 0.8) (drill 0.2) (layers "F.Cu" "B.Cu") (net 5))
 (via (at 93.175666 87.432446) (size 0.8) (drill 0.2) (layers "F.Cu" "B.Cu") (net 5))
 (via (at 94.234 90.395777) (size 0.8) (drill 0.2) (layers "F.Cu" "B.Cu") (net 5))
 (via (at 91.059 88.420223) (size 0.8) (drill 0.2) (layers "F.Cu" "B.Cu") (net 5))
 (via (at 94.234 89.408) (size 0.8) (drill 0.2) (layers "F.Cu" "B.Cu") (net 5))
 (via (at 92.117333 90.395777) (size 0.8) (drill 0.2) (layers "F.Cu" "B.Cu") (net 5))
 (via (at 92.117333 87.432446) (size 0.8) (drill 0.2) (layers "F.Cu" "B.Cu") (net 5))
 (segment (start 94.352 92.193) (end 94.615 92.456) (width 0.25) (layer "F.Cu") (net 1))
 (segment (start 91.1835 92.8395) (end 91.83 92.193) (width 0.25) (layer "F.Cu") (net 1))
 (segment (start 94.615 99.314) (end 94.361 99.568) (width 0.25) (layer "F.Cu") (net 1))
 (segment (start 94.615 92.456) (end 94.615 99.314) (width 0.25) (layer "F.Cu") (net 1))
 (segment (start 94.361 99.568) (end 92.182 99.568) (width 0.25) (layer "F.Cu") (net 1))
 (segment (start 91.1835 93.218) (end 91.1835 92.8395) (width 0.25) (layer "F.Cu") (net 1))
 (segment (start 91.83 92.193) (end 94.352 92.193) (width 0.25) (layer "F.Cu") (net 1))
 (segment (start 93.2335 95.3295) (end 93.186 95.377) (width 1.15) (layer "F.Cu") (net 2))
 (segment (start 93.2335 93.218) (end 93.2335 95.3295) (width 1.15) (layer "F.Cu") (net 2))
 (segment (start 88.539 78.596) (end 88.539 79.228) (width 1.15) (layer "F.Cu") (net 6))
 (segment (start 89.798 84.709) (end 89.798 79.855) (width 1.15) (layer "F.Cu") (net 6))
 (segment (start 89.798 79.855) (end 88.539 78.596) (width 1.15) (layer "F.Cu") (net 6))
 (segment (start 88.539 79.228) (end 89.829 80.518) (width 1.15) (layer "F.Cu") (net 6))
 (segment (start 88.9 95.2975) (end 88.9 98.786) (width 1.15) (layer "F.Cu") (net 7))
 (segment (start 91.1065 95.2975) (end 91.186 95.377) (width 1.15) (layer "F.Cu") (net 7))
 (segment (start 88.9 95.2975) (end 91.1065 95.2975) (width 1.15) (layer "F.Cu") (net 7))
 (segment (start 88.9 98.786) (end 89.682 99.568) (width 1.15) (layer "F.Cu") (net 7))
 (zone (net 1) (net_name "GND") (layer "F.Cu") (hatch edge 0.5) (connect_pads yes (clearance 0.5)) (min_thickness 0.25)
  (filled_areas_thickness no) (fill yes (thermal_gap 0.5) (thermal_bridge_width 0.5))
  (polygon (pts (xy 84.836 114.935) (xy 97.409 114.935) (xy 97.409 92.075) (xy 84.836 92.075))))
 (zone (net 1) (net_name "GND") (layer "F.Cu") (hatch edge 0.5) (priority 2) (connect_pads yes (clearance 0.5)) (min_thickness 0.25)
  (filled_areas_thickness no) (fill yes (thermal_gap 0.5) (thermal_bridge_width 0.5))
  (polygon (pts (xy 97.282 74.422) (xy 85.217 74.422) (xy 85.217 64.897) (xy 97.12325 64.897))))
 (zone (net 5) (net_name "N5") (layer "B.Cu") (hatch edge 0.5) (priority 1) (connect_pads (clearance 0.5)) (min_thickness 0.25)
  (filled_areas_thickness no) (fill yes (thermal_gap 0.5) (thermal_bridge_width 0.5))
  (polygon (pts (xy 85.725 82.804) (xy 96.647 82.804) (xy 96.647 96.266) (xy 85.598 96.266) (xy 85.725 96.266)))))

